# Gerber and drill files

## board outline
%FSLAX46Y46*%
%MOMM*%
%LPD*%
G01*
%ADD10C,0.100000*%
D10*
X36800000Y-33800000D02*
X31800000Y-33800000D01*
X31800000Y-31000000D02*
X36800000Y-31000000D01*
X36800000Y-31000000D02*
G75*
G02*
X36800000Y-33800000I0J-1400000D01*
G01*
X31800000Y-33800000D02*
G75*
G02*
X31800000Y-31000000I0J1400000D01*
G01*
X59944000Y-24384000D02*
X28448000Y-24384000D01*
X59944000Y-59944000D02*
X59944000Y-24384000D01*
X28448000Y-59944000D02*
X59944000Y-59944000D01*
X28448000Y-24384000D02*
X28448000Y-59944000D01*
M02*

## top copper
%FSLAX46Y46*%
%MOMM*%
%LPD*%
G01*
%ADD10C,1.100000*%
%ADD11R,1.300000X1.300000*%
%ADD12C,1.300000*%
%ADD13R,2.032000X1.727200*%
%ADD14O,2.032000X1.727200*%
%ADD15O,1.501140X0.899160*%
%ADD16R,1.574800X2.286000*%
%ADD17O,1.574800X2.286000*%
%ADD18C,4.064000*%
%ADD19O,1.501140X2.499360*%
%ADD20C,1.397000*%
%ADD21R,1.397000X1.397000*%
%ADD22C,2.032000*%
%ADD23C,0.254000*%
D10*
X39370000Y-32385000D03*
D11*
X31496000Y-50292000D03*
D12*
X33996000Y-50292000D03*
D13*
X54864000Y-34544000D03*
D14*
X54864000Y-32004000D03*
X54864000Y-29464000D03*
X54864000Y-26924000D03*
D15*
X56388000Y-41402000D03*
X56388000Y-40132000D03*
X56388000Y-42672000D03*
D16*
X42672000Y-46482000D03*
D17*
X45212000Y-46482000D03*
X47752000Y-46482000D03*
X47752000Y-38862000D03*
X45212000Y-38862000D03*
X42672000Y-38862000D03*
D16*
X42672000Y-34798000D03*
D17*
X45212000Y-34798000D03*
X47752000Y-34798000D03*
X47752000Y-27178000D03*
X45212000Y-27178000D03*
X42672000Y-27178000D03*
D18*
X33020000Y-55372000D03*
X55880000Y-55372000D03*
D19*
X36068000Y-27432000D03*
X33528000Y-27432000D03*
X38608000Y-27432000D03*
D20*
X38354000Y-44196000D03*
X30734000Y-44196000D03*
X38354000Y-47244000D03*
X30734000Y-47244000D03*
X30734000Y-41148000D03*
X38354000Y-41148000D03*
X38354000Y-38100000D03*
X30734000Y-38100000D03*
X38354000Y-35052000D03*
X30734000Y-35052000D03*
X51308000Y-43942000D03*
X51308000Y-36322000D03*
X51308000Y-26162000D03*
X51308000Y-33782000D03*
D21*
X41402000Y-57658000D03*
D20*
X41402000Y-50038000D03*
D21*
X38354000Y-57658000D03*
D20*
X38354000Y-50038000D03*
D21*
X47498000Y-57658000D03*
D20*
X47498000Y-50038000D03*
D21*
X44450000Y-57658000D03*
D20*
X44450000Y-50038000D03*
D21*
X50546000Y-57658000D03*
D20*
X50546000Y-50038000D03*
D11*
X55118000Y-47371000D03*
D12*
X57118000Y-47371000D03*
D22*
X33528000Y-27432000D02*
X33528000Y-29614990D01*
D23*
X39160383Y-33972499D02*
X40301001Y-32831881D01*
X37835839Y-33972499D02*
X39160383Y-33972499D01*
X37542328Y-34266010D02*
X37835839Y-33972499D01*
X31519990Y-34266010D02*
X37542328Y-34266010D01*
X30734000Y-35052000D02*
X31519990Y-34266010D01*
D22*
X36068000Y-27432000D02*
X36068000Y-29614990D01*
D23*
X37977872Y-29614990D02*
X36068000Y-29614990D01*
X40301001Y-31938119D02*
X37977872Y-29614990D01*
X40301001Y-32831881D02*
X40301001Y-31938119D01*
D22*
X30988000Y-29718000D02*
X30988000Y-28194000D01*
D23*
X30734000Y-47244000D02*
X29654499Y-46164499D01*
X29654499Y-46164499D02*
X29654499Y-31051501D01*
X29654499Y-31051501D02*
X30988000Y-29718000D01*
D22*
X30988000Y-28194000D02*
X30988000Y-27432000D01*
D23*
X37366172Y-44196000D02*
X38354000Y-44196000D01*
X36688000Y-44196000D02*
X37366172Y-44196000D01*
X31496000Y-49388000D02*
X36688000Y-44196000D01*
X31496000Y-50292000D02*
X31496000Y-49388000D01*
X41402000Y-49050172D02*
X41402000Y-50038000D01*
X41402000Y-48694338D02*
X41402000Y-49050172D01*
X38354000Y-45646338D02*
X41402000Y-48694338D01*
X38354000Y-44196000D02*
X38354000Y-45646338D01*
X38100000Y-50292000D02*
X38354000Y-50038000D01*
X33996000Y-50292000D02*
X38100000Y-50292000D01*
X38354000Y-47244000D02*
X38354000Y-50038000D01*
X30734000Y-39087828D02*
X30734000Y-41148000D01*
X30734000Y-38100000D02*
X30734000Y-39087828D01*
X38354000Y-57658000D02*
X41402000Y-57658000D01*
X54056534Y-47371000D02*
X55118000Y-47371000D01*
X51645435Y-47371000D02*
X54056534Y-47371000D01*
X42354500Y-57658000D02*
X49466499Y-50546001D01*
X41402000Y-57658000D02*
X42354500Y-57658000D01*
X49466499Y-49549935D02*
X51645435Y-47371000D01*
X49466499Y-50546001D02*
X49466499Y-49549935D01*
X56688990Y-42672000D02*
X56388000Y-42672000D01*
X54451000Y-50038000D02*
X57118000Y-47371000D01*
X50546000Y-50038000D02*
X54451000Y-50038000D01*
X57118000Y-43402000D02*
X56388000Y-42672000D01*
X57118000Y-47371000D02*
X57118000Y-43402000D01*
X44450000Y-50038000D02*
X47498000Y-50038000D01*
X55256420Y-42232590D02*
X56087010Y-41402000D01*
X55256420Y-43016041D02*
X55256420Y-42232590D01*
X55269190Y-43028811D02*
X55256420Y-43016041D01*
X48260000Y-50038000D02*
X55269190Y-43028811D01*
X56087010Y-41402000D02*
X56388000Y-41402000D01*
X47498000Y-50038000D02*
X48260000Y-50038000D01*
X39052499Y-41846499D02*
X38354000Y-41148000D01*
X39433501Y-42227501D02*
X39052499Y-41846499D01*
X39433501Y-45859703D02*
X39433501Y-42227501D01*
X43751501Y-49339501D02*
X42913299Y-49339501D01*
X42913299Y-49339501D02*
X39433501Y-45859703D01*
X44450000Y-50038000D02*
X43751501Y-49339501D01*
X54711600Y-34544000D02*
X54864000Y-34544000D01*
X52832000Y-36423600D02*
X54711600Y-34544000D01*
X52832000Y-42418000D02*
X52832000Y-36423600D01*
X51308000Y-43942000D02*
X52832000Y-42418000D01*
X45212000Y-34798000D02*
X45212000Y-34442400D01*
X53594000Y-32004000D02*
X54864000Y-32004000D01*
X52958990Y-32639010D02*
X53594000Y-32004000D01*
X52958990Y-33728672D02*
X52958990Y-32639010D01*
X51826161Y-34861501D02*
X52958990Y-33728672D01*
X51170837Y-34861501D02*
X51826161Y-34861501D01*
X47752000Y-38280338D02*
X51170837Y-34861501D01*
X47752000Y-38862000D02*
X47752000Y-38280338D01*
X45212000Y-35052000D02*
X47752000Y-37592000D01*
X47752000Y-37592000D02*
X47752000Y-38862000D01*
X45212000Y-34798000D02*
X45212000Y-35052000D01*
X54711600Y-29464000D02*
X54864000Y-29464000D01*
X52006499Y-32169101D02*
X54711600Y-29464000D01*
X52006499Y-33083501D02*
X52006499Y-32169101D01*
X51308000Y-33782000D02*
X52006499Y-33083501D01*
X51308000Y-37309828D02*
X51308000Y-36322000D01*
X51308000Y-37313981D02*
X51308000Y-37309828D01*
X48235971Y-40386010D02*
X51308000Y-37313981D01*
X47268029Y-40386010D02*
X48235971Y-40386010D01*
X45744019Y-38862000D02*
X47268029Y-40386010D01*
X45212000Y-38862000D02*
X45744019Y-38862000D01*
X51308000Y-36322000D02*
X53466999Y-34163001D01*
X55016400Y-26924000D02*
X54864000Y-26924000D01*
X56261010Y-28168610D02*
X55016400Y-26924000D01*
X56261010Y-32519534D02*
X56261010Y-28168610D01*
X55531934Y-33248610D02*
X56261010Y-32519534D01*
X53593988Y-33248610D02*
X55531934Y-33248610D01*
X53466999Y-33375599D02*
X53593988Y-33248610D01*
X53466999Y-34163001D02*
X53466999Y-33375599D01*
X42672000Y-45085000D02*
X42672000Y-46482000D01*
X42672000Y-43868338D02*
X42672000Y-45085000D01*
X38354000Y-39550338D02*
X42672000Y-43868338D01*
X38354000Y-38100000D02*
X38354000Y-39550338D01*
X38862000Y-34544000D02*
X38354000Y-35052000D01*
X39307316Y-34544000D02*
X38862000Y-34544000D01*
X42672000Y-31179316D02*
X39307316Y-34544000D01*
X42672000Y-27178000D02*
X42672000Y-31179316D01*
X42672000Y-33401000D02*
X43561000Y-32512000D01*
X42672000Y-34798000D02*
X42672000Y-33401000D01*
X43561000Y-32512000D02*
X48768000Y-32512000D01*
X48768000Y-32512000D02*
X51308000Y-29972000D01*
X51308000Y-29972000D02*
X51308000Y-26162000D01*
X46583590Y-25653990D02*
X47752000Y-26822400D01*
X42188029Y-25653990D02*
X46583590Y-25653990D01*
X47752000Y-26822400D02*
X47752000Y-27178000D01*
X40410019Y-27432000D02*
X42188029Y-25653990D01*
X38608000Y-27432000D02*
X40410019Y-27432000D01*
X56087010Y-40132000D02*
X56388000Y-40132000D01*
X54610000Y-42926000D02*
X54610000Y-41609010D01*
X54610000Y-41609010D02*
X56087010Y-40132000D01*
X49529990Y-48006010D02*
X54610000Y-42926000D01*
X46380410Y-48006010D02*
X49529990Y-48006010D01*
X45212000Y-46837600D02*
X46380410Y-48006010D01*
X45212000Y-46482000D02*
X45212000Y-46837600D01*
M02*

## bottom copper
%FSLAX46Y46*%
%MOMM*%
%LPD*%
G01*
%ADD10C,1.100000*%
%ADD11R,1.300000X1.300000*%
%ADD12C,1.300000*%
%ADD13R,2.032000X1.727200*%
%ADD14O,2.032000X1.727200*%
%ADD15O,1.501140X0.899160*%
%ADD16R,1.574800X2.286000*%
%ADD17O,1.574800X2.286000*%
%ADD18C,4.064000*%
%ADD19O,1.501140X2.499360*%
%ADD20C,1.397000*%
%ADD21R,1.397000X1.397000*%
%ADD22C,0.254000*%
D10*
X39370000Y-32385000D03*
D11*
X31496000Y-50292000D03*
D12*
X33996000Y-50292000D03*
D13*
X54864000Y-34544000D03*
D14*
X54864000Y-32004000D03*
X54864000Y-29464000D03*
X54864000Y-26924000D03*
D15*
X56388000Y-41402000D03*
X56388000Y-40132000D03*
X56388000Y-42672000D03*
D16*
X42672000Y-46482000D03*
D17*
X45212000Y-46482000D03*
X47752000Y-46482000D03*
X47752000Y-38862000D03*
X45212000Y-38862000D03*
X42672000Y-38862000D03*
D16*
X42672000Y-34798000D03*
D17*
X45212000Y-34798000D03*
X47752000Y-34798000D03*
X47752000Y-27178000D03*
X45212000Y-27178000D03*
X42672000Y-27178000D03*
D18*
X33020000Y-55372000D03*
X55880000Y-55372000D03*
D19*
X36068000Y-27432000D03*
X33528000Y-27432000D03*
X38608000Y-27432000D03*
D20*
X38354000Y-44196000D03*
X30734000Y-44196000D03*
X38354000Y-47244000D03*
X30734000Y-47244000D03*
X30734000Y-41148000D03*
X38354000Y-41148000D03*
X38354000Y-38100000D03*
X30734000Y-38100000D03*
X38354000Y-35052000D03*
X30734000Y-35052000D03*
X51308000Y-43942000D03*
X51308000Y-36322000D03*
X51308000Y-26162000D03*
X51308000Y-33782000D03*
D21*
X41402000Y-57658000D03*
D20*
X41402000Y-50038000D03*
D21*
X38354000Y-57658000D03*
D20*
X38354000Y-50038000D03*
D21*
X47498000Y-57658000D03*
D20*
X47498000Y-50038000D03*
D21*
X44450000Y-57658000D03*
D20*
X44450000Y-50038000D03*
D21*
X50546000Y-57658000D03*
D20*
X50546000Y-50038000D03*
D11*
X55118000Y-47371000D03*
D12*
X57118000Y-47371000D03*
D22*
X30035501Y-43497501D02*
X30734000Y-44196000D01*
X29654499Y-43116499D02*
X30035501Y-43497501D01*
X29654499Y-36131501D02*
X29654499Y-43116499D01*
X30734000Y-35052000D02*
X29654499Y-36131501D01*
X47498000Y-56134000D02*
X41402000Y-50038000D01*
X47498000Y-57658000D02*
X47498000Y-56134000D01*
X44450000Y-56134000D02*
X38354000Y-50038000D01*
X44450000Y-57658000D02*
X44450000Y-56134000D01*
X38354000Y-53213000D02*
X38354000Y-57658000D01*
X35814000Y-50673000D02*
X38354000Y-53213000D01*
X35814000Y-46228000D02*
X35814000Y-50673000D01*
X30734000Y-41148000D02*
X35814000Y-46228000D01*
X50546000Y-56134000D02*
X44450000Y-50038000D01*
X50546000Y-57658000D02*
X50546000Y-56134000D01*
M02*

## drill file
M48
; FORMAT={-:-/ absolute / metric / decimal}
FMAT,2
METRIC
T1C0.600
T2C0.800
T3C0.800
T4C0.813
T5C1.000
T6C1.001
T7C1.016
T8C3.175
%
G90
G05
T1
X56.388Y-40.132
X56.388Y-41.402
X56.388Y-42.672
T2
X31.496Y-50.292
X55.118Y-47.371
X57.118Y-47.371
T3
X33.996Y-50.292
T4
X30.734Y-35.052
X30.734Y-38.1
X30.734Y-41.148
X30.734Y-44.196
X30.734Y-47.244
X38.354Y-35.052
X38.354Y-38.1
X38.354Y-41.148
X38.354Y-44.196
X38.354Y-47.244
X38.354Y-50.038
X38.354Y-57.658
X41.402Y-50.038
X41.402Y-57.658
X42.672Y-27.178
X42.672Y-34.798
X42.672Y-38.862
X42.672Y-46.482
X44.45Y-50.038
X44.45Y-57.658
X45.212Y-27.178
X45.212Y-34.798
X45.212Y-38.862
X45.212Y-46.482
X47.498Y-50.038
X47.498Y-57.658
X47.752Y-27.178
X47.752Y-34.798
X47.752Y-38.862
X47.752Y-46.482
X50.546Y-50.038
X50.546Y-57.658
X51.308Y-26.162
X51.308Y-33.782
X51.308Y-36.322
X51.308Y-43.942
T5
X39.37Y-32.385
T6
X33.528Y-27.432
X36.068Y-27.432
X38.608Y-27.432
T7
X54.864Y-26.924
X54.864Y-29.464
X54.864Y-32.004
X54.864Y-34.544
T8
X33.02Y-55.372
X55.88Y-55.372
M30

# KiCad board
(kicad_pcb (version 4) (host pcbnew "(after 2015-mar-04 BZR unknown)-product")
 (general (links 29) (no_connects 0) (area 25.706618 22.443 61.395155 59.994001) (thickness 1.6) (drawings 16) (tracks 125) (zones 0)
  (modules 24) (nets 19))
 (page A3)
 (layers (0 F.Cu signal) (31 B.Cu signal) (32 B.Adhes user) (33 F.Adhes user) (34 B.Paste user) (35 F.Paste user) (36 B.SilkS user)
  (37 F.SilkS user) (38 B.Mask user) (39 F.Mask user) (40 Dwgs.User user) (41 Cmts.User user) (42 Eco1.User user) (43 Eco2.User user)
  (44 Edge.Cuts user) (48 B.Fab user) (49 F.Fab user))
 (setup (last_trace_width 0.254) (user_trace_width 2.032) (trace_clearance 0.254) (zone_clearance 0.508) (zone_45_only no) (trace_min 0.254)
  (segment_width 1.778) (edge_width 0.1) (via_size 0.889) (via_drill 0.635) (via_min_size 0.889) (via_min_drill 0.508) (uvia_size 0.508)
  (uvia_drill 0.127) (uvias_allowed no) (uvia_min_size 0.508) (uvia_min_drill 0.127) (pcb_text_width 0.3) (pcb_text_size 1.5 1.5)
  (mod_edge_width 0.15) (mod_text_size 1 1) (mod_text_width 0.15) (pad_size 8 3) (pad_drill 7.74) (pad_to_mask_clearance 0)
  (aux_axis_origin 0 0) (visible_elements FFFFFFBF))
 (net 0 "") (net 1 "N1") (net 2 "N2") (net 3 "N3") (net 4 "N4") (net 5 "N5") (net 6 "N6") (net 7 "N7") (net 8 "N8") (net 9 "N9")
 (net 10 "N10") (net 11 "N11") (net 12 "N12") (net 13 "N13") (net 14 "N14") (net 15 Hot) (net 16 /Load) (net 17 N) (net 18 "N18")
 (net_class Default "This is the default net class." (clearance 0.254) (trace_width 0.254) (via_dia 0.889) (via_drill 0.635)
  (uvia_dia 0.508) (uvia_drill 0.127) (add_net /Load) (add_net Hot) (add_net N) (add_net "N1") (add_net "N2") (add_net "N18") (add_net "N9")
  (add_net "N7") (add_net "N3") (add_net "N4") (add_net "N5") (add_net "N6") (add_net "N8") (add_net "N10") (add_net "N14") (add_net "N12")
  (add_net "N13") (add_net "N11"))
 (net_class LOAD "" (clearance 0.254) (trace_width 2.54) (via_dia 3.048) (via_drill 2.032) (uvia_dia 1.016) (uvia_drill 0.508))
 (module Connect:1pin (layer F.Cu) (at 39.37 32.385)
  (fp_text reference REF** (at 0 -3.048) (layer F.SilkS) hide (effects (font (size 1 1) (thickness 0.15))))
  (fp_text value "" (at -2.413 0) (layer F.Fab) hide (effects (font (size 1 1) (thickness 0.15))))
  (pad "" thru_hole circle (at 0 0) (size 1.1 1.1) (drill 1) (layers *.Cu *.Mask F.SilkS)))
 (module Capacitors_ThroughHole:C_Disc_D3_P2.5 (layer F.Cu) (at 31.496 50.292)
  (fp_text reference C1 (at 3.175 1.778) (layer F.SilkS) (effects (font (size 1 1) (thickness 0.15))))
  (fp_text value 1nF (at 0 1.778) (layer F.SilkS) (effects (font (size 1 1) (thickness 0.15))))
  (pad 1 thru_hole rect (at 0 0) (size 1.3 1.3) (drill 0.8) (layers *.Cu *.Mask F.SilkS) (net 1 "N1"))
  (pad 2 thru_hole circle (at 2.5 0) (size 1.3 1.3) (drill 0.8001) (layers *.Cu *.Mask F.SilkS) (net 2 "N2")))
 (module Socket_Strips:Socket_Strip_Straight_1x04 (layer F.Cu) (at 54.864 34.544 90)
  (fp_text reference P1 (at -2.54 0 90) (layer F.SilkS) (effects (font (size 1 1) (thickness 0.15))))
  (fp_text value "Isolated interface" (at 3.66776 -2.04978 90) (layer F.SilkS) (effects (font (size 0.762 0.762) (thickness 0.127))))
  (pad 1 thru_hole rect (at 0 0 90) (size 1.7272 2.032) (drill 1.016) (layers *.Cu *.Mask F.SilkS) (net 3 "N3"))
  (pad 2 thru_hole oval (at 2.54 0 90) (size 1.7272 2.032) (drill 1.016) (layers *.Cu *.Mask F.SilkS) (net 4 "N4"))
  (pad 3 thru_hole oval (at 5.08 0 90) (size 1.7272 2.032) (drill 1.016) (layers *.Cu *.Mask F.SilkS) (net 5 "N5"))
  (pad 4 thru_hole oval (at 7.62 0 90) (size 1.7272 2.032) (drill 1.016) (layers *.Cu *.Mask F.SilkS) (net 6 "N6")))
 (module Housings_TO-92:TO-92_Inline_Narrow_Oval (layer F.Cu) (at 56.388 42.672 90)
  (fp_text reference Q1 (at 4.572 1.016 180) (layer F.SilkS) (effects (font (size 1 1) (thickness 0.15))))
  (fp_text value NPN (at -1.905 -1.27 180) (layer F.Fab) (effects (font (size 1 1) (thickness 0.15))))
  (pad 2 thru_hole oval (at 1.27 0 270) (size 0.89916 1.50114) (drill 0.6) (layers *.Cu *.Mask F.SilkS) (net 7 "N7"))
  (pad 3 thru_hole oval (at 2.54 0 270) (size 0.89916 1.50114) (drill 0.6) (layers *.Cu *.Mask F.SilkS) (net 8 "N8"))
  (pad 1 thru_hole oval (at 0 0 270) (size 0.89916 1.50114) (drill 0.6) (layers *.Cu *.Mask F.SilkS) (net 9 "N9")))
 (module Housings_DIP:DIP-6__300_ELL (layer F.Cu) (at 45.212 42.672)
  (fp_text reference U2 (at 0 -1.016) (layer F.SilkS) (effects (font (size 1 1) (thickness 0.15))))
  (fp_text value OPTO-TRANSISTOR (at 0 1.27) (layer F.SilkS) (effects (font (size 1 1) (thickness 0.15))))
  (pad 1 thru_hole rect (at -2.54 3.81) (size 1.5748 2.286) (drill 0.8128) (layers *.Cu *.Mask F.SilkS) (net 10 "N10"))
  (pad 2 thru_hole oval (at 0 3.81) (size 1.5748 2.286) (drill 0.8128) (layers *.Cu *.Mask F.SilkS) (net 8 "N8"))
  (pad 3 thru_hole oval (at 2.54 3.81) (size 1.5748 2.286) (drill 0.8128) (layers *.Cu *.Mask F.SilkS))
  (pad 4 thru_hole oval (at 2.54 -3.81) (size 1.5748 2.286) (drill 0.8128) (layers *.Cu *.Mask F.SilkS) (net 4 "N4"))
  (pad 5 thru_hole oval (at 0 -3.81) (size 1.5748 2.286) (drill 0.8128) (layers *.Cu *.Mask F.SilkS) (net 6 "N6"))
  (pad 6 thru_hole oval (at -2.54 -3.81) (size 1.5748 2.286) (drill 0.8128) (layers *.Cu *.Mask F.SilkS) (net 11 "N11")))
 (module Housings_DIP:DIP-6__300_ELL (layer F.Cu) (at 45.212 30.988)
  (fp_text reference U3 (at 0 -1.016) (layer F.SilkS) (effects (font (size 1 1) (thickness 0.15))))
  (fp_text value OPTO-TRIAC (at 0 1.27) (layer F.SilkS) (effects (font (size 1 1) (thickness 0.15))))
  (pad 1 thru_hole rect (at -2.54 3.81) (size 1.5748 2.286) (drill 0.8128) (layers *.Cu *.Mask F.SilkS) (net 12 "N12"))
  (pad 2 thru_hole oval (at 0 3.81) (size 1.5748 2.286) (drill 0.8128) (layers *.Cu *.Mask F.SilkS) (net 4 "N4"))
  (pad 3 thru_hole oval (at 2.54 3.81) (size 1.5748 2.286) (drill 0.8128) (layers *.Cu *.Mask F.SilkS))
  (pad 4 thru_hole oval (at 2.54 -3.81) (size 1.5748 2.286) (drill 0.8128) (layers *.Cu *.Mask F.SilkS) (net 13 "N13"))
  (pad 5 thru_hole oval (at 0 -3.81) (size 1.5748 2.286) (drill 0.8128) (layers *.Cu *.Mask F.SilkS))
  (pad 6 thru_hole oval (at -2.54 -3.81) (size 1.5748 2.286) (drill 0.8128) (layers *.Cu *.Mask F.SilkS) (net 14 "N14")))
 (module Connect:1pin (layer F.Cu) (at 33.02 55.372)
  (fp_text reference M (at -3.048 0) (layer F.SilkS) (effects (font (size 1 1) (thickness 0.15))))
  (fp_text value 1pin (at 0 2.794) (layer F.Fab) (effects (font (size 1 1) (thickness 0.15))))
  (pad 1 thru_hole circle (at 0 0) (size 4.064 4.064) (drill 3.175) (layers *.Cu *.Mask F.SilkS)))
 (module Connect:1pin (layer F.Cu) (at 55.88 55.372)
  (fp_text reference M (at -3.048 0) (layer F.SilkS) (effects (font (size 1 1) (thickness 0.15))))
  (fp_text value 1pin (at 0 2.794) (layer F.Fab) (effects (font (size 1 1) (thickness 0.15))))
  (pad 1 thru_hole circle (at 0 0) (size 4.064 4.064) (drill 3.175) (layers *.Cu *.Mask F.SilkS)))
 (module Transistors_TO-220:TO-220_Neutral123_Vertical (layer B.Cu) (at 36.068 27.432)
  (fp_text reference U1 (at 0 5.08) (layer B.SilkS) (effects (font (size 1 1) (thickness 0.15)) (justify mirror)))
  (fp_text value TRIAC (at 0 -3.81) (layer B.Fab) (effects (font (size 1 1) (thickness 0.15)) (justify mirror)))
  (pad 2 thru_hole oval (at 0 0 270) (size 2.49936 1.50114) (drill 1.00076) (layers *.Cu *.Mask B.SilkS) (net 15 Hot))
  (pad 1 thru_hole oval (at -2.54 0 270) (size 2.49936 1.50114) (drill 1.00076) (layers *.Cu *.Mask B.SilkS) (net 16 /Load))
  (pad 3 thru_hole oval (at 2.54 0 270) (size 2.49936 1.50114) (drill 1.00076) (layers *.Cu *.Mask B.SilkS) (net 13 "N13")))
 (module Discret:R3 (layer F.Cu) (at 34.544 44.196 180)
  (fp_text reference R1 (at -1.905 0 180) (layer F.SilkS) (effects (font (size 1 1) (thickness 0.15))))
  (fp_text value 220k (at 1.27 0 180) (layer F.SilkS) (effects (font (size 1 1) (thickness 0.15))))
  (pad 1 thru_hole circle (at -3.81 0 180) (size 1.397 1.397) (drill 0.8128) (layers *.Cu *.Mask F.SilkS) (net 1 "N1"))
  (pad 2 thru_hole circle (at 3.81 0 180) (size 1.397 1.397) (drill 0.8128) (layers *.Cu *.Mask F.SilkS) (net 15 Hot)))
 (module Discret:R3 (layer F.Cu) (at 34.544 47.244 180)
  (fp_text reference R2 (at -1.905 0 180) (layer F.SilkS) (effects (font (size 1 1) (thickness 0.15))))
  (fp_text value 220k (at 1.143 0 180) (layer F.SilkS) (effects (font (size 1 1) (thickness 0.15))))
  (pad 1 thru_hole circle (at -3.81 0 180) (size 1.397 1.397) (drill 0.8128) (layers *.Cu *.Mask F.SilkS) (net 2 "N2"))
  (pad 2 thru_hole circle (at 3.81 0 180) (size 1.397 1.397) (drill 0.8128) (layers *.Cu *.Mask F.SilkS) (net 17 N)))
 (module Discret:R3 (layer F.Cu) (at 34.544 41.148)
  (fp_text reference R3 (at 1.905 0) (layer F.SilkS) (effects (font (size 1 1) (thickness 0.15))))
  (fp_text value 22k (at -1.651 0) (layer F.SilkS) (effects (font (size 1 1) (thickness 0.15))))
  (pad 1 thru_hole circle (at -3.81 0) (size 1.397 1.397) (drill 0.8128) (layers *.Cu *.Mask F.SilkS) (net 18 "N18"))
  (pad 2 thru_hole circle (at 3.81 0) (size 1.397 1.397) (drill 0.8128) (layers *.Cu *.Mask F.SilkS) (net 7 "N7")))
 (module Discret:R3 (layer F.Cu) (at 34.544 38.1 180)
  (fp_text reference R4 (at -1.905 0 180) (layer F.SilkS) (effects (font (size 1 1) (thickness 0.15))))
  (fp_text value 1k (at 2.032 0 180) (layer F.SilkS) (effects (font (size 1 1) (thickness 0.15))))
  (pad 1 thru_hole circle (at -3.81 0 180) (size 1.397 1.397) (drill 0.8128) (layers *.Cu *.Mask F.SilkS) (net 10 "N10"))
  (pad 2 thru_hole circle (at 3.81 0 180) (size 1.397 1.397) (drill 0.8128) (layers *.Cu *.Mask F.SilkS) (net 18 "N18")))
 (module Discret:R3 (layer F.Cu) (at 34.544 35.052 180)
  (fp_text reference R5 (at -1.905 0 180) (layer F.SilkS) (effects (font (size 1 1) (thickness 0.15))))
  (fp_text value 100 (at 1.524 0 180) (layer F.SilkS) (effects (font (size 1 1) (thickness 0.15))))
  (pad 1 thru_hole circle (at -3.81 0 180) (size 1.397 1.397) (drill 0.8128) (layers *.Cu *.Mask F.SilkS) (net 14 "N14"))
  (pad 2 thru_hole circle (at 3.81 0 180) (size 1.397 1.397) (drill 0.8128) (layers *.Cu *.Mask F.SilkS) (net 15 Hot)))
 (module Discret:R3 (layer F.Cu) (at 51.308 40.132 90)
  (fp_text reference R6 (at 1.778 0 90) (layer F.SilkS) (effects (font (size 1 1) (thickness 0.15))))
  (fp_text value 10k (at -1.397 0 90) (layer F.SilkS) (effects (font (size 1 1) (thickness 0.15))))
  (pad 1 thru_hole circle (at -3.81 0 90) (size 1.397 1.397) (drill 0.8128) (layers *.Cu *.Mask F.SilkS) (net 3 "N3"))
  (pad 2 thru_hole circle (at 3.81 0 90) (size 1.397 1.397) (drill 0.8128) (layers *.Cu *.Mask F.SilkS) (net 6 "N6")))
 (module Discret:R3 (layer F.Cu) (at 51.308 29.972 270)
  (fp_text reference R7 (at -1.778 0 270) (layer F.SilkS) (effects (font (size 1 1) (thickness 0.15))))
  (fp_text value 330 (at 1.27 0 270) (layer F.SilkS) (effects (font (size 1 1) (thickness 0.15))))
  (pad 1 thru_hole circle (at -3.81 0 270) (size 1.397 1.397) (drill 0.8128) (layers *.Cu *.Mask F.SilkS) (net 12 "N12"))
  (pad 2 thru_hole circle (at 3.81 0 270) (size 1.397 1.397) (drill 0.8128) (layers *.Cu *.Mask F.SilkS) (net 5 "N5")))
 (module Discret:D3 (layer F.Cu) (at 41.402 53.848 270)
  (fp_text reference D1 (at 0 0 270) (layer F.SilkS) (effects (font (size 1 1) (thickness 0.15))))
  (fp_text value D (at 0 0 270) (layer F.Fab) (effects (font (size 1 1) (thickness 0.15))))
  (pad 2 thru_hole rect (at 3.81 0 270) (size 1.397 1.397) (drill 0.8128) (layers *.Cu *.Mask F.SilkS) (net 18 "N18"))
  (pad 1 thru_hole circle (at -3.81 0 270) (size 1.397 1.397) (drill 0.8128) (layers *.Cu *.Mask F.SilkS) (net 1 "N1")))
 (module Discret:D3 (layer F.Cu) (at 38.354 53.848 270)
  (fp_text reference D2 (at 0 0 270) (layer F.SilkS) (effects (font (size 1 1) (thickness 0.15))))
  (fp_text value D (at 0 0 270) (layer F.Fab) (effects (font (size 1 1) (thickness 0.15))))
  (pad 2 thru_hole rect (at 3.81 0 270) (size 1.397 1.397) (drill 0.8128) (layers *.Cu *.Mask F.SilkS) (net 18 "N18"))
  (pad 1 thru_hole circle (at -3.81 0 270) (size 1.397 1.397) (drill 0.8128) (layers *.Cu *.Mask F.SilkS) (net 2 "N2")))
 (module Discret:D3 (layer F.Cu) (at 47.498 53.848 270)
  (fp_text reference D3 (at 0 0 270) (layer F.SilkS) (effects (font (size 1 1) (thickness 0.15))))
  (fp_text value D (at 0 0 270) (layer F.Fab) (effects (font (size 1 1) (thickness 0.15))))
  (pad 2 thru_hole rect (at 3.81 0 270) (size 1.397 1.397) (drill 0.8128) (layers *.Cu *.Mask F.SilkS) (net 1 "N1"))
  (pad 1 thru_hole circle (at -3.81 0 270) (size 1.397 1.397) (drill 0.8128) (layers *.Cu *.Mask F.SilkS) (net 7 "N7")))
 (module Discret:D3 (layer F.Cu) (at 44.45 53.848 270)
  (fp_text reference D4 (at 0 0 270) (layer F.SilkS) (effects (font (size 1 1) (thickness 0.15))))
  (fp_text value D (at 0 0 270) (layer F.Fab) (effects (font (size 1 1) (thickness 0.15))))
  (pad 2 thru_hole rect (at 3.81 0 270) (size 1.397 1.397) (drill 0.8128) (layers *.Cu *.Mask F.SilkS) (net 2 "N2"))
  (pad 1 thru_hole circle (at -3.81 0 270) (size 1.397 1.397) (drill 0.8128) (layers *.Cu *.Mask F.SilkS) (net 7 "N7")))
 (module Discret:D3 (layer F.Cu) (at 50.546 53.848 270)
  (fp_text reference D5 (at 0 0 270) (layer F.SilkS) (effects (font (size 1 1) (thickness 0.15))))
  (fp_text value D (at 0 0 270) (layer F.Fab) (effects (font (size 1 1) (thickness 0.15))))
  (pad 2 thru_hole rect (at 3.81 0 270) (size 1.397 1.397) (drill 0.8128) (layers *.Cu *.Mask F.SilkS) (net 7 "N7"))
  (pad 1 thru_hole circle (at -3.81 0 270) (size 1.397 1.397) (drill 0.8128) (layers *.Cu *.Mask F.SilkS) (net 9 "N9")))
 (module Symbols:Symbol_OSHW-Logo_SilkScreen (layer B.Cu) (at 42.672 53.848 270)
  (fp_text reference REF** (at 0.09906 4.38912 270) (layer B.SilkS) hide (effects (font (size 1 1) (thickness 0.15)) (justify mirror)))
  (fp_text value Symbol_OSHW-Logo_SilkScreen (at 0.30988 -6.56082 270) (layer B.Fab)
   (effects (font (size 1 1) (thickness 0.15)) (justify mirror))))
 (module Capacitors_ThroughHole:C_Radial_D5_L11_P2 (layer F.Cu) (at 55.118 47.371)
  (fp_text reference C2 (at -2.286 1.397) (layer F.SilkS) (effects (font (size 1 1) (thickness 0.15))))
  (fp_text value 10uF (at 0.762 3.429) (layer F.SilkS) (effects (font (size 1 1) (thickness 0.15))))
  (pad 1 thru_hole rect (at 0 0) (size 1.3 1.3) (drill 0.8) (layers *.Cu *.Mask F.SilkS) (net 18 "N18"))
  (pad 2 thru_hole circle (at 2 0) (size 1.3 1.3) (drill 0.8) (layers *.Cu *.Mask F.SilkS) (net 9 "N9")))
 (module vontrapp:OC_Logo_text (layer B.Cu) (at 34.544 38.1 270)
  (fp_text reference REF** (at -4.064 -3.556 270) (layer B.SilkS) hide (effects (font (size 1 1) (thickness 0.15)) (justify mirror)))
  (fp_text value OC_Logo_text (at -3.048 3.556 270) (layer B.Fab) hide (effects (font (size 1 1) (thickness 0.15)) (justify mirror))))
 (gr_line (start 36.8 33.8) (end 31.8 33.8) (angle 90) (layer Edge.Cuts) (width 0.1))
 (gr_line (start 31.8 31) (end 36.8 31) (angle 90) (layer Edge.Cuts) (width 0.1))
 (gr_arc (start 36.8 32.4) (end 36.8 31) (angle 180) (layer Edge.Cuts) (width 0.1))
 (gr_arc (start 31.8 32.4) (end 31.8 33.8) (angle 180) (layer Edge.Cuts) (width 0.1))
 (gr_line (start 59.944 24.384) (end 28.448 24.384) (angle 90) (layer Edge.Cuts) (width 0.1))
 (gr_line (start 59.944 59.944) (end 59.944 24.384) (angle 90) (layer Edge.Cuts) (width 0.1))
 (gr_line (start 28.448 59.944) (end 59.944 59.944) (angle 90) (layer Edge.Cuts) (width 0.1))
 (gr_line (start 28.448 24.384) (end 28.448 59.944) (angle 90) (layer Edge.Cuts) (width 0.1))
 (segment (start 33.528 27.432) (end 33.528 29.61499) (width 2.032) (layer F.Cu) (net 16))
 (segment (start 39.160383 33.972499) (end 40.301001 32.831881) (width 0.254) (layer F.Cu) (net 15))
 (segment (start 37.835839 33.972499) (end 39.160383 33.972499) (width 0.254) (layer F.Cu) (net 15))
 (segment (start 37.542328 34.26601) (end 37.835839 33.972499) (width 0.254) (layer F.Cu) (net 15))
 (segment (start 31.51999 34.26601) (end 37.542328 34.26601) (width 0.254) (layer F.Cu) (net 15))
 (segment (start 30.734 35.052) (end 31.51999 34.26601) (width 0.254) (layer F.Cu) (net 15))
 (segment (start 30.035501 43.497501) (end 30.734 44.196) (width 0.254) (layer B.Cu) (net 15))
 (segment (start 29.654499 43.116499) (end 30.035501 43.497501) (width 0.254) (layer B.Cu) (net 15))
 (segment (start 29.654499 36.131501) (end 29.654499 43.116499) (width 0.254) (layer B.Cu) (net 15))
 (segment (start 30.734 35.052) (end 29.654499 36.131501) (width 0.254) (layer B.Cu) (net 15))
 (segment (start 36.068 27.432) (end 36.068 29.61499) (width 2.032) (layer F.Cu) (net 15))
 (segment (start 37.977872 29.61499) (end 36.068 29.61499) (width 0.254) (layer F.Cu) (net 15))
 (segment (start 40.301001 31.938119) (end 37.977872 29.61499) (width 0.254) (layer F.Cu) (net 15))
 (segment (start 40.301001 32.831881) (end 40.301001 31.938119) (width 0.254) (layer F.Cu) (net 15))
 (segment (start 30.988 29.718) (end 30.988 28.194) (width 2.032) (layer F.Cu) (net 17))
 (segment (start 30.734 47.244) (end 29.654499 46.164499) (width 0.254) (layer F.Cu) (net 17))
 (segment (start 29.654499 46.164499) (end 29.654499 31.051501) (width 0.254) (layer F.Cu) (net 17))
 (segment (start 29.654499 31.051501) (end 30.988 29.718) (width 0.254) (layer F.Cu) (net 17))
 (segment (start 30.988 28.194) (end 30.988 27.432) (width 2.032) (layer F.Cu) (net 17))
 (segment (start 37.366172 44.196) (end 38.354 44.196) (width 0.254) (layer F.Cu) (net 1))
 (segment (start 36.688 44.196) (end 37.366172 44.196) (width 0.254) (layer F.Cu) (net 1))
 (segment (start 31.496 49.388) (end 36.688 44.196) (width 0.254) (layer F.Cu) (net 1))
 (segment (start 31.496 50.292) (end 31.496 49.388) (width 0.254) (layer F.Cu) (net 1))
 (segment (start 41.402 49.050172) (end 41.402 50.038) (width 0.254) (layer F.Cu) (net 1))
 (segment (start 41.402 48.694338) (end 41.402 49.050172) (width 0.254) (layer F.Cu) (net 1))
 (segment (start 38.354 45.646338) (end 41.402 48.694338) (width 0.254) (layer F.Cu) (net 1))
 (segment (start 38.354 44.196) (end 38.354 45.646338) (width 0.254) (layer F.Cu) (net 1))
 (segment (start 47.498 56.134) (end 41.402 50.038) (width 0.254) (layer B.Cu) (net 1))
 (segment (start 47.498 57.658) (end 47.498 56.134) (width 0.254) (layer B.Cu) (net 1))
 (segment (start 38.1 50.292) (end 38.354 50.038) (width 0.254) (layer F.Cu) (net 2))
 (segment (start 33.996 50.292) (end 38.1 50.292) (width 0.254) (layer F.Cu) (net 2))
 (segment (start 38.354 47.244) (end 38.354 50.038) (width 0.254) (layer F.Cu) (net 2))
 (segment (start 44.45 56.134) (end 38.354 50.038) (width 0.254) (layer B.Cu) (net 2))
 (segment (start 44.45 57.658) (end 44.45 56.134) (width 0.254) (layer B.Cu) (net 2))
 (segment (start 30.734 39.087828) (end 30.734 41.148) (width 0.254) (layer F.Cu) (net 18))
 (segment (start 30.734 38.1) (end 30.734 39.087828) (width 0.254) (layer F.Cu) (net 18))
 (segment (start 38.354 57.658) (end 41.402 57.658) (width 0.254) (layer F.Cu) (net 18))
 (segment (start 54.056534 47.371) (end 55.118 47.371) (width 0.254) (layer F.Cu) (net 18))
 (segment (start 51.645435 47.371) (end 54.056534 47.371) (width 0.254) (layer F.Cu) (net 18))
 (segment (start 42.3545 57.658) (end 49.466499 50.546001) (width 0.254) (layer F.Cu) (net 18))
 (segment (start 41.402 57.658) (end 42.3545 57.658) (width 0.254) (layer F.Cu) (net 18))
 (segment (start 49.466499 49.549935) (end 51.645435 47.371) (width 0.254) (layer F.Cu) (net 18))
 (segment (start 49.466499 50.546001) (end 49.466499 49.549935) (width 0.254) (layer F.Cu) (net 18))
 (segment (start 38.354 53.213) (end 38.354 57.658) (width 0.254) (layer B.Cu) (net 18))
 (segment (start 35.814 50.673) (end 38.354 53.213) (width 0.254) (layer B.Cu) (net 18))
 (segment (start 35.814 46.228) (end 35.814 50.673) (width 0.254) (layer B.Cu) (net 18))
 (segment (start 30.734 41.148) (end 35.814 46.228) (width 0.254) (layer B.Cu) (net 18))
 (segment (start 56.68899 42.672) (end 56.388 42.672) (width 0.254) (layer F.Cu) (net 9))
 (segment (start 54.451 50.038) (end 57.118 47.371) (width 0.254) (layer F.Cu) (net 9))
 (segment (start 50.546 50.038) (end 54.451 50.038) (width 0.254) (layer F.Cu) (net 9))
 (segment (start 57.118 43.402) (end 56.388 42.672) (width 0.254) (layer F.Cu) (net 9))
 (segment (start 57.118 47.371) (end 57.118 43.402) (width 0.254) (layer F.Cu) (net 9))
 (segment (start 50.546 56.134) (end 44.45 50.038) (width 0.254) (layer B.Cu) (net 7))
 (segment (start 50.546 57.658) (end 50.546 56.134) (width 0.254) (layer B.Cu) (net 7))
 (segment (start 44.45 50.038) (end 47.498 50.038) (width 0.254) (layer F.Cu) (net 7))
 (segment (start 55.25642 42.23259) (end 56.08701 41.402) (width 0.254) (layer F.Cu) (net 7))
 (segment (start 55.25642 43.016041) (end 55.25642 42.23259) (width 0.254) (layer F.Cu) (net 7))
 (segment (start 55.26919 43.028811) (end 55.25642 43.016041) (width 0.254) (layer F.Cu) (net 7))
 (segment (start 48.26 50.038) (end 55.26919 43.028811) (width 0.254) (layer F.Cu) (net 7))
 (segment (start 56.08701 41.402) (end 56.388 41.402) (width 0.254) (layer F.Cu) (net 7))
 (segment (start 47.498 50.038) (end 48.26 50.038) (width 0.254) (layer F.Cu) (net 7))
 (segment (start 39.052499 41.846499) (end 38.354 41.148) (width 0.254) (layer F.Cu) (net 7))
 (segment (start 39.433501 42.227501) (end 39.052499 41.846499) (width 0.254) (layer F.Cu) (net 7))
 (segment (start 39.433501 45.859703) (end 39.433501 42.227501) (width 0.254) (layer F.Cu) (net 7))
 (segment (start 43.751501 49.339501) (end 42.913299 49.339501) (width 0.254) (layer F.Cu) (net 7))
 (segment (start 42.913299 49.339501) (end 39.433501 45.859703) (width 0.254) (layer F.Cu) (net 7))
 (segment (start 44.45 50.038) (end 43.751501 49.339501) (width 0.254) (layer F.Cu) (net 7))
 (segment (start 54.7116 34.544) (end 54.864 34.544) (width 0.254) (layer F.Cu) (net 3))
 (segment (start 52.832 36.4236) (end 54.7116 34.544) (width 0.254) (layer F.Cu) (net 3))
 (segment (start 52.832 42.418) (end 52.832 36.4236) (width 0.254) (layer F.Cu) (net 3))
 (segment (start 51.308 43.942) (end 52.832 42.418) (width 0.254) (layer F.Cu) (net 3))
 (segment (start 45.212 34.798) (end 45.212 34.4424) (width 0.254) (layer F.Cu) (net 4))
 (segment (start 53.594 32.004) (end 54.864 32.004) (width 0.254) (layer F.Cu) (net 4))
 (segment (start 52.95899 32.63901) (end 53.594 32.004) (width 0.254) (layer F.Cu) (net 4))
 (segment (start 52.95899 33.728672) (end 52.95899 32.63901) (width 0.254) (layer F.Cu) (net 4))
 (segment (start 51.826161 34.861501) (end 52.95899 33.728672) (width 0.254) (layer F.Cu) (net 4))
 (segment (start 51.170837 34.861501) (end 51.826161 34.861501) (width 0.254) (layer F.Cu) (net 4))
 (segment (start 47.752 38.280338) (end 51.170837 34.861501) (width 0.254) (layer F.Cu) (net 4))
 (segment (start 47.752 38.862) (end 47.752 38.280338) (width 0.254) (layer F.Cu) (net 4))
 (segment (start 45.212 35.052) (end 47.752 37.592) (width 0.254) (layer F.Cu) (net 4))
 (segment (start 47.752 37.592) (end 47.752 38.862) (width 0.254) (layer F.Cu) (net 4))
 (segment (start 45.212 34.798) (end 45.212 35.052) (width 0.254) (layer F.Cu) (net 4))
 (segment (start 54.7116 29.464) (end 54.864 29.464) (width 0.254) (layer F.Cu) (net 5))
 (segment (start 52.006499 32.169101) (end 54.7116 29.464) (width 0.254) (layer F.Cu) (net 5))
 (segment (start 52.006499 33.083501) (end 52.006499 32.169101) (width 0.254) (layer F.Cu) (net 5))
 (segment (start 51.308 33.782) (end 52.006499 33.083501) (width 0.254) (layer F.Cu) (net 5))
 (segment (start 51.308 37.309828) (end 51.308 36.322) (width 0.254) (layer F.Cu) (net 6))
 (segment (start 51.308 37.313981) (end 51.308 37.309828) (width 0.254) (layer F.Cu) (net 6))
 (segment (start 48.235971 40.38601) (end 51.308 37.313981) (width 0.254) (layer F.Cu) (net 6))
 (segment (start 47.268029 40.38601) (end 48.235971 40.38601) (width 0.254) (layer F.Cu) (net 6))
 (segment (start 45.744019 38.862) (end 47.268029 40.38601) (width 0.254) (layer F.Cu) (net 6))
 (segment (start 45.212 38.862) (end 45.744019 38.862) (width 0.254) (layer F.Cu) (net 6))
 (segment (start 51.308 36.322) (end 53.466999 34.163001) (width 0.254) (layer F.Cu) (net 6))
 (segment (start 55.0164 26.924) (end 54.864 26.924) (width 0.254) (layer F.Cu) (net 6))
 (segment (start 56.26101 28.16861) (end 55.0164 26.924) (width 0.254) (layer F.Cu) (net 6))
 (segment (start 56.26101 32.519534) (end 56.26101 28.16861) (width 0.254) (layer F.Cu) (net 6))
 (segment (start 55.531934 33.24861) (end 56.26101 32.519534) (width 0.254) (layer F.Cu) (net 6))
 (segment (start 53.593988 33.24861) (end 55.531934 33.24861) (width 0.254) (layer F.Cu) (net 6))
 (segment (start 53.466999 33.375599) (end 53.593988 33.24861) (width 0.254) (layer F.Cu) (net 6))
 (segment (start 53.466999 34.163001) (end 53.466999 33.375599) (width 0.254) (layer F.Cu) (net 6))
 (segment (start 42.672 45.085) (end 42.672 46.482) (width 0.254) (layer F.Cu) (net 10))
 (segment (start 42.672 43.868338) (end 42.672 45.085) (width 0.254) (layer F.Cu) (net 10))
 (segment (start 38.354 39.550338) (end 42.672 43.868338) (width 0.254) (layer F.Cu) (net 10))
 (segment (start 38.354 38.1) (end 38.354 39.550338) (width 0.254) (layer F.Cu) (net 10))
 (segment (start 38.862 34.544) (end 38.354 35.052) (width 0.254) (layer F.Cu) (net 14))
 (segment (start 39.307316 34.544) (end 38.862 34.544) (width 0.254) (layer F.Cu) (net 14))
 (segment (start 42.672 31.179316) (end 39.307316 34.544) (width 0.254) (layer F.Cu) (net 14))
 (segment (start 42.672 27.178) (end 42.672 31.179316) (width 0.254) (layer F.Cu) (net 14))
 (segment (start 42.672 33.401) (end 43.561 32.512) (width 0.254) (layer F.Cu) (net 12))
 (segment (start 42.672 34.798) (end 42.672 33.401) (width 0.254) (layer F.Cu) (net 12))
 (segment (start 43.561 32.512) (end 48.768 32.512) (width 0.254) (layer F.Cu) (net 12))
 (segment (start 48.768 32.512) (end 51.308 29.972) (width 0.254) (layer F.Cu) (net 12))
 (segment (start 51.308 29.972) (end 51.308 26.162) (width 0.254) (layer F.Cu) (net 12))
 (segment (start 46.58359 25.65399) (end 47.752 26.8224) (width 0.254) (layer F.Cu) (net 13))
 (segment (start 42.188029 25.65399) (end 46.58359 25.65399) (width 0.254) (layer F.Cu) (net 13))
 (segment (start 47.752 26.8224) (end 47.752 27.178) (width 0.254) (layer F.Cu) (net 13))
 (segment (start 40.410019 27.432) (end 42.188029 25.65399) (width 0.254) (layer F.Cu) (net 13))
 (segment (start 38.608 27.432) (end 40.410019 27.432) (width 0.254) (layer F.Cu) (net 13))
 (segment (start 56.08701 40.132) (end 56.388 40.132) (width 0.254) (layer F.Cu) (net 8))
 (segment (start 54.61 42.926) (end 54.61 41.60901) (width 0.254) (layer F.Cu) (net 8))
 (segment (start 54.61 41.60901) (end 56.08701 40.132) (width 0.254) (layer F.Cu) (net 8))
 (segment (start 49.52999 48.00601) (end 54.61 42.926) (width 0.254) (layer F.Cu) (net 8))
 (segment (start 46.38041 48.00601) (end 49.52999 48.00601) (width 0.254) (layer F.Cu) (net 8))
 (segment (start 45.212 46.8376) (end 46.38041 48.00601) (width 0.254) (layer F.Cu) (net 8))
 (segment (start 45.212 46.482) (end 45.212 46.8376) (width 0.254) (layer F.Cu) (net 8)))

